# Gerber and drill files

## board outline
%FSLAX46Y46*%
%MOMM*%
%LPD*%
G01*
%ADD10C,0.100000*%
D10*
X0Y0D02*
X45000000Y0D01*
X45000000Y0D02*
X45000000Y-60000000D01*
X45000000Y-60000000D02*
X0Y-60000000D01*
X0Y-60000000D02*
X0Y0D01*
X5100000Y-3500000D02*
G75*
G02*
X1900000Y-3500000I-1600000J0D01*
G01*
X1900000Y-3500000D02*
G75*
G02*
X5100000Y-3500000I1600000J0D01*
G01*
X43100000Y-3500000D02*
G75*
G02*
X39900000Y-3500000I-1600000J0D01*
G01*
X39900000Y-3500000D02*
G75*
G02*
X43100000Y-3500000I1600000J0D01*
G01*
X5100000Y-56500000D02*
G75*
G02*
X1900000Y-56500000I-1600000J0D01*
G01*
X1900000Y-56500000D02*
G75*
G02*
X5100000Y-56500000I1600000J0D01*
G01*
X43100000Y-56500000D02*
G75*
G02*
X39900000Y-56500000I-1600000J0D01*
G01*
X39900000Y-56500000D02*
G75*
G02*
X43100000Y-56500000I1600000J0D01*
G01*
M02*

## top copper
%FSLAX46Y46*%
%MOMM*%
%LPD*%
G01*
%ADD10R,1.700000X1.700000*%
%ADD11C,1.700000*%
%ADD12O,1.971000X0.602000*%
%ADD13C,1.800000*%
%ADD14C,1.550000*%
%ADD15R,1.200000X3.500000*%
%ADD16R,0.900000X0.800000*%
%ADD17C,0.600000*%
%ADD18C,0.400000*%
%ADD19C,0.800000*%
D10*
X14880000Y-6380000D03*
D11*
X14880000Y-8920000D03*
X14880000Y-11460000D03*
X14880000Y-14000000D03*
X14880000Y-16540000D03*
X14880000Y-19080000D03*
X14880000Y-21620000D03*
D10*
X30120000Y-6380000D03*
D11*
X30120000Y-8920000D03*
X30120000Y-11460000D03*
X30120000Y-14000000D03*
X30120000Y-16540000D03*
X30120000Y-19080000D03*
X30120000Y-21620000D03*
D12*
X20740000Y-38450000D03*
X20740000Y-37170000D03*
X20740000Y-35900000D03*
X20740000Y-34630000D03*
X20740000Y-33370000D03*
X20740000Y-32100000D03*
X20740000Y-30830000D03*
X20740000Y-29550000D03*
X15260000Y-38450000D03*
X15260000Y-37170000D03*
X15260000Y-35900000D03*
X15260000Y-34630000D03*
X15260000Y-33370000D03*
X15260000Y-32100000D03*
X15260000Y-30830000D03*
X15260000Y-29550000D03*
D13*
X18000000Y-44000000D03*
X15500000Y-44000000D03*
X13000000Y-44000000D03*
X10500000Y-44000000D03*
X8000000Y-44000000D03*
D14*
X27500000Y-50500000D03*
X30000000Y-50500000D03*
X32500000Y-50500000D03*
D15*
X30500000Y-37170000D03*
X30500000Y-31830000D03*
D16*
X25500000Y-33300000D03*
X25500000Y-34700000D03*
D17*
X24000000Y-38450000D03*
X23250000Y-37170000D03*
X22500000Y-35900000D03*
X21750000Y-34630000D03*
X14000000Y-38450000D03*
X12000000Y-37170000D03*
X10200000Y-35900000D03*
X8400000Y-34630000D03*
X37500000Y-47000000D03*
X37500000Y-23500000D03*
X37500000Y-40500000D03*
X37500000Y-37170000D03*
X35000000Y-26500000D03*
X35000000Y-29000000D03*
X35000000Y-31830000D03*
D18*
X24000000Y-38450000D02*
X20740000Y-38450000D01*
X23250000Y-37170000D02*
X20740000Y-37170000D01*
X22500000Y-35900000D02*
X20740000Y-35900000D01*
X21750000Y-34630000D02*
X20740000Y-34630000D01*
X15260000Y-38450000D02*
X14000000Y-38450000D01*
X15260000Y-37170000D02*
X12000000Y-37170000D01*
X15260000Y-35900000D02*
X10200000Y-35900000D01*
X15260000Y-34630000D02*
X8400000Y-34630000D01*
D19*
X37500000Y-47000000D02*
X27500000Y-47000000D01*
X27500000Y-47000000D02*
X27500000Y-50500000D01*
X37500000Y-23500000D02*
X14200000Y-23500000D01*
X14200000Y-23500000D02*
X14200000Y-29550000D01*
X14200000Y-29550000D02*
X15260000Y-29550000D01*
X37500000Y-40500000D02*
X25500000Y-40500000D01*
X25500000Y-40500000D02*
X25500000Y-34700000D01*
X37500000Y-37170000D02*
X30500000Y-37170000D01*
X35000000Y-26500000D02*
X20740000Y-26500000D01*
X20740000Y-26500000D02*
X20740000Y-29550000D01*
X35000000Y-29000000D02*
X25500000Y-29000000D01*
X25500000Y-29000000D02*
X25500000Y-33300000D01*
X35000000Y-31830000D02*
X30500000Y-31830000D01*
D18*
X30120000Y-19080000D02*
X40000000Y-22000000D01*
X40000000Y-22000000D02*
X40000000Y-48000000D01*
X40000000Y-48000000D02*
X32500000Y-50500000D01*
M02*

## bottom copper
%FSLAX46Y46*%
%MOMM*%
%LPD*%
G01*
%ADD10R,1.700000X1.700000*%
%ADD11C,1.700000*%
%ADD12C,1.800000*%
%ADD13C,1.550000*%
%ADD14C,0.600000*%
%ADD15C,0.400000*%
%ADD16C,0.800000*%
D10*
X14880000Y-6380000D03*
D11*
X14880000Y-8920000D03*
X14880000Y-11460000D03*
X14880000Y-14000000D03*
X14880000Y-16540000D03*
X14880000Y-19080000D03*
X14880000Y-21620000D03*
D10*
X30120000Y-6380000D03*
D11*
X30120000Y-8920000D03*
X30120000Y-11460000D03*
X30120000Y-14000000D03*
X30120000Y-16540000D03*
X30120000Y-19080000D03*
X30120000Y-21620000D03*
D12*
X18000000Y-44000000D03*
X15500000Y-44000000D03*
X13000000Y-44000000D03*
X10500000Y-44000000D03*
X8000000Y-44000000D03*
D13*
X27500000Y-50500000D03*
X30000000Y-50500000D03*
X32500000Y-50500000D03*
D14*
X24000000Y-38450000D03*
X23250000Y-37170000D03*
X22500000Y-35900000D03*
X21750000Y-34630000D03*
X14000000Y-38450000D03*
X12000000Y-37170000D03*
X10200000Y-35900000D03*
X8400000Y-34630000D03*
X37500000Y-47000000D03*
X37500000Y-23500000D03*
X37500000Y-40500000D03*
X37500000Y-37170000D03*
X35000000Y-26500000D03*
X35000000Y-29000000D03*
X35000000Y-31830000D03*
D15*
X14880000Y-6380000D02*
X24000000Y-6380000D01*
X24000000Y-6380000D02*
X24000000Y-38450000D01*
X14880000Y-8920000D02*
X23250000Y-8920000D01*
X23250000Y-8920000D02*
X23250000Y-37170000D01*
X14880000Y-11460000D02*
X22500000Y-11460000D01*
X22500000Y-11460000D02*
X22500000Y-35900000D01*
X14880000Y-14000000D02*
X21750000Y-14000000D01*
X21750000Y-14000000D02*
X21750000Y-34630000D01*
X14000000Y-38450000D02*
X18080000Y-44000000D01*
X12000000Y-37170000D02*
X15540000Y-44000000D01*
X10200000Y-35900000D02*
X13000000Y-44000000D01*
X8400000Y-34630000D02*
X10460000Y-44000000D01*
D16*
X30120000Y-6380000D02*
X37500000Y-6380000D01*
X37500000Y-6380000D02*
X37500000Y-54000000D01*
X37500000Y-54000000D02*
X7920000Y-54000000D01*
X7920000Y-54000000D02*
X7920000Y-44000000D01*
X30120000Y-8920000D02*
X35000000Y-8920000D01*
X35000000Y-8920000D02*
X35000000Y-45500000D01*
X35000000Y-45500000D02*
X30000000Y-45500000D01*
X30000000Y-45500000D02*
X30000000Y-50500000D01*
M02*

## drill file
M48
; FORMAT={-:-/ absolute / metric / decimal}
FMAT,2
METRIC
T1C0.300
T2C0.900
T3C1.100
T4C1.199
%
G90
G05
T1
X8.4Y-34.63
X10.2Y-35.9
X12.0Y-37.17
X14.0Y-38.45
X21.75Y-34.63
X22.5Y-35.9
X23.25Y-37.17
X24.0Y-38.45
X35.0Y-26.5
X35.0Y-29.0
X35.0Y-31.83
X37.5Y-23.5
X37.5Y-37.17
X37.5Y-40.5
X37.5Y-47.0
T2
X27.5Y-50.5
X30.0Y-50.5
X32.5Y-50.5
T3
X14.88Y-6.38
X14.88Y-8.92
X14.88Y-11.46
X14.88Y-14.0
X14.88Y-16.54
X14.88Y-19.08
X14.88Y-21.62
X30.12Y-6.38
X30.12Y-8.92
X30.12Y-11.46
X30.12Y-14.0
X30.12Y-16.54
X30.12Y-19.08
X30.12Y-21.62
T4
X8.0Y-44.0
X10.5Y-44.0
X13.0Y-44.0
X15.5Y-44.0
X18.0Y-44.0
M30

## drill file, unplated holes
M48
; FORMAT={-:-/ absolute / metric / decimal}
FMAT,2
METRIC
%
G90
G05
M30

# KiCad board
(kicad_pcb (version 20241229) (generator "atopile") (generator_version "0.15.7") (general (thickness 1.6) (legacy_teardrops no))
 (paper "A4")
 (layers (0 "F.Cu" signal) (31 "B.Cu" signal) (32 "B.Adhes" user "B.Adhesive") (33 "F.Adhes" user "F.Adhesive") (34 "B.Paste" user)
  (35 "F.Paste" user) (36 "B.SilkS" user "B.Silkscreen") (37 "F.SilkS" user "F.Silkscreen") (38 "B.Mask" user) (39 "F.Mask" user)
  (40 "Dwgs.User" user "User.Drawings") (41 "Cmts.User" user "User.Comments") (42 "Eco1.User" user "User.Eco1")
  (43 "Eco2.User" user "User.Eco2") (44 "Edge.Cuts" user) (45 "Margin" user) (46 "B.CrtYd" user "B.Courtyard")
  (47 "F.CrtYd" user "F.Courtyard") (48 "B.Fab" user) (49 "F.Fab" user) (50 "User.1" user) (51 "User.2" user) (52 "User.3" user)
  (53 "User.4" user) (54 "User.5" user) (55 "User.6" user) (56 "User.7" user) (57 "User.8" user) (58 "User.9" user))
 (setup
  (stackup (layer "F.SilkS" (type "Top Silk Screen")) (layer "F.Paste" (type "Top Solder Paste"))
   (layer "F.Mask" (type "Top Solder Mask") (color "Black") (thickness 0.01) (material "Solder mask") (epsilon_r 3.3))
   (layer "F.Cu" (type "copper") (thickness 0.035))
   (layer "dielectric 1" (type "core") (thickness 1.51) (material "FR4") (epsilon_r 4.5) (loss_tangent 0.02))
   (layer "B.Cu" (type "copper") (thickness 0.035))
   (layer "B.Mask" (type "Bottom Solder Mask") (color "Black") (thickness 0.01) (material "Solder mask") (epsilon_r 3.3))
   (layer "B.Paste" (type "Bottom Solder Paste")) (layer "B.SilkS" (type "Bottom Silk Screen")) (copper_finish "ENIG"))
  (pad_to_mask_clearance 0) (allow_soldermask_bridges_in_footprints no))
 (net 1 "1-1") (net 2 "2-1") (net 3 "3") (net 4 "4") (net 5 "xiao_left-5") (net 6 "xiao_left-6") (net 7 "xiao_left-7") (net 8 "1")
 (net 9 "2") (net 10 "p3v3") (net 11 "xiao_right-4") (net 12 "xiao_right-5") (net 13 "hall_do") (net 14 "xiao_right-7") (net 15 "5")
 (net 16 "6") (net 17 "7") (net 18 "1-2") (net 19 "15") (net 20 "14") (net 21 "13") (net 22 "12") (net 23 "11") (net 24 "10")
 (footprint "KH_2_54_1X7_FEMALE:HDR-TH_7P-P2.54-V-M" (layer "F.Cu") (at 14.88 14 270)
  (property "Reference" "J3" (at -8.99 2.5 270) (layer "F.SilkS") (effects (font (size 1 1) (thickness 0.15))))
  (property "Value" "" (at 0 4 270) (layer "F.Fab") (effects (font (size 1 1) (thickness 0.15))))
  (pad "1" thru_hole rect (at -7.62 0 270) (size 1.7 1.7) (drill 1.100024) (layers "*.Cu" "*.Mask") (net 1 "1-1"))
  (pad "2" thru_hole circle (at -5.08 0 270) (size 1.7 1.7) (drill 1.100024) (layers "*.Cu" "*.Mask") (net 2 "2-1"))
  (pad "3" thru_hole circle (at -2.54 0 270) (size 1.7 1.7) (drill 1.100024) (layers "*.Cu" "*.Mask") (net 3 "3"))
  (pad "4" thru_hole circle (at 0 0 270) (size 1.7 1.7) (drill 1.100024) (layers "*.Cu" "*.Mask") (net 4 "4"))
  (pad "5" thru_hole circle (at 2.54 0 270) (size 1.7 1.7) (drill 1.100024) (layers "*.Cu" "*.Mask") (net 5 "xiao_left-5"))
  (pad "6" thru_hole circle (at 5.08 0 270) (size 1.7 1.7) (drill 1.100024) (layers "*.Cu" "*.Mask") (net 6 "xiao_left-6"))
  (pad "7" thru_hole circle (at 7.62 0 270) (size 1.7 1.7) (drill 1.100024) (layers "*.Cu" "*.Mask") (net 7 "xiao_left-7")))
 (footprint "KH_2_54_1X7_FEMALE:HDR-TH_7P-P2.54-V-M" (layer "F.Cu") (at 30.12 14 270)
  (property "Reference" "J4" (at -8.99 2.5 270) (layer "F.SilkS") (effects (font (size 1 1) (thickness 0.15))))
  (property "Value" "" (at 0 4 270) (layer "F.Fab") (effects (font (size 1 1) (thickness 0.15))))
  (pad "1" thru_hole rect (at -7.62 0 270) (size 1.7 1.7) (drill 1.100024) (layers "*.Cu" "*.Mask") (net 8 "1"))
  (pad "2" thru_hole circle (at -5.08 0 270) (size 1.7 1.7) (drill 1.100024) (layers "*.Cu" "*.Mask") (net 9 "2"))
  (pad "3" thru_hole circle (at -2.54 0 270) (size 1.7 1.7) (drill 1.100024) (layers "*.Cu" "*.Mask") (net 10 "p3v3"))
  (pad "4" thru_hole circle (at 0 0 270) (size 1.7 1.7) (drill 1.100024) (layers "*.Cu" "*.Mask") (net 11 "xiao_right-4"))
  (pad "5" thru_hole circle (at 2.54 0 270) (size 1.7 1.7) (drill 1.100024) (layers "*.Cu" "*.Mask") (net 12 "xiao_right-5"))
  (pad "6" thru_hole circle (at 5.08 0 270) (size 1.7 1.7) (drill 1.100024) (layers "*.Cu" "*.Mask") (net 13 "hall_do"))
  (pad "7" thru_hole circle (at 7.62 0 270) (size 1.7 1.7) (drill 1.100024) (layers "*.Cu" "*.Mask") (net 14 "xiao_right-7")))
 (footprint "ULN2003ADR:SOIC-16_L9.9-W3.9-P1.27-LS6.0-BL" (layer "F.Cu") (at 18 34 90)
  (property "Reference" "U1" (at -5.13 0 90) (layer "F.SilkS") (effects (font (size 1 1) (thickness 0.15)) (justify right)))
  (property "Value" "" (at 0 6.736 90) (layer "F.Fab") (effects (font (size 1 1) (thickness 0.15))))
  (pad "1" smd oval (at -4.45 2.74 90) (size 0.602 1.971) (layers "F.Cu" "F.Paste" "F.Mask") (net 1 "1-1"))
  (pad "2" smd oval (at -3.17 2.74 90) (size 0.602 1.971) (layers "F.Cu" "F.Paste" "F.Mask") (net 2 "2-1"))
  (pad "3" smd oval (at -1.9 2.74 90) (size 0.602 1.971) (layers "F.Cu" "F.Paste" "F.Mask") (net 3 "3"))
  (pad "4" smd oval (at -0.63 2.74 90) (size 0.602 1.971) (layers "F.Cu" "F.Paste" "F.Mask") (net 4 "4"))
  (pad "5" smd oval (at 0.63 2.74 90) (size 0.602 1.971) (layers "F.Cu" "F.Paste" "F.Mask") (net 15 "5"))
  (pad "6" smd oval (at 1.9 2.74 90) (size 0.602 1.971) (layers "F.Cu" "F.Paste" "F.Mask") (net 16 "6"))
  (pad "7" smd oval (at 3.17 2.74 90) (size 0.602 1.971) (layers "F.Cu" "F.Paste" "F.Mask") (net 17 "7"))
  (pad "8" smd oval (at 4.45 2.74 90) (size 0.602 1.971) (layers "F.Cu" "F.Paste" "F.Mask") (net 9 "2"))
  (pad "16" smd oval (at -4.45 -2.74 90) (size 0.602 1.971) (layers "F.Cu" "F.Paste" "F.Mask") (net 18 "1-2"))
  (pad "15" smd oval (at -3.17 -2.74 90) (size 0.602 1.971) (layers "F.Cu" "F.Paste" "F.Mask") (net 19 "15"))
  (pad "14" smd oval (at -1.9 -2.74 90) (size 0.602 1.971) (layers "F.Cu" "F.Paste" "F.Mask") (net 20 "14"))
  (pad "13" smd oval (at -0.63 -2.74 90) (size 0.602 1.971) (layers "F.Cu" "F.Paste" "F.Mask") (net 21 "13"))
  (pad "12" smd oval (at 0.63 -2.74 90) (size 0.602 1.971) (layers "F.Cu" "F.Paste" "F.Mask") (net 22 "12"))
  (pad "11" smd oval (at 1.9 -2.74 90) (size 0.602 1.971) (layers "F.Cu" "F.Paste" "F.Mask") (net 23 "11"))
  (pad "10" smd oval (at 3.17 -2.74 90) (size 0.602 1.971) (layers "F.Cu" "F.Paste" "F.Mask") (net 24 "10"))
  (pad "9" smd oval (at 4.45 -2.74 90) (size 0.602 1.971) (layers "F.Cu" "F.Paste" "F.Mask") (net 8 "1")))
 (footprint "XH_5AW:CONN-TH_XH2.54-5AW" (layer "F.Cu") (at 13 44 0)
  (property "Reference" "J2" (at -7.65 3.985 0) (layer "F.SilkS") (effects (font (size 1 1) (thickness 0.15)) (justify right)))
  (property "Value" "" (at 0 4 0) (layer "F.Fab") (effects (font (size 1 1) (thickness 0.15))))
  (pad "1" thru_hole circle (at 5 -0 180) (size 1.8 1.8) (drill 1.19888) (layers "*.Cu" "*.Mask") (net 18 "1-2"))
  (pad "2" thru_hole circle (at 2.5 -0 180) (size 1.8 1.8) (drill 1.19888) (layers "*.Cu" "*.Mask") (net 19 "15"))
  (pad "3" thru_hole circle (at -0 -0 180) (size 1.8 1.8) (drill 1.19888) (layers "*.Cu" "*.Mask") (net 20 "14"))
  (pad "4" thru_hole circle (at -2.5 -0 180) (size 1.8 1.8) (drill 1.19888) (layers "*.Cu" "*.Mask") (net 21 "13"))
  (pad "5" thru_hole circle (at -5 -0 180) (size 1.8 1.8) (drill 1.19888) (layers "*.Cu" "*.Mask") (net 8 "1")))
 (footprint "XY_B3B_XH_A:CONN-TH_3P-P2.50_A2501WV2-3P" (layer "F.Cu") (at 30 50.5 0)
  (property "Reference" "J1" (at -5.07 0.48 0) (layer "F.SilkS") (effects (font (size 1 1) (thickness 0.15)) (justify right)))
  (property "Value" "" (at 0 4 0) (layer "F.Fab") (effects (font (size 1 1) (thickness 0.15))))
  (pad "1" thru_hole circle (at -2.5 0 180) (size 1.55 1.55) (drill 0.900024) (layers "*.Cu" "*.Mask") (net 8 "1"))
  (pad "2" thru_hole circle (at 0 0 180) (size 1.55 1.55) (drill 0.900024) (layers "*.Cu" "*.Mask") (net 9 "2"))
  (pad "3" thru_hole circle (at 2.5 0 180) (size 1.55 1.55) (drill 0.900024) (layers "*.Cu" "*.Mask") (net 13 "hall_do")))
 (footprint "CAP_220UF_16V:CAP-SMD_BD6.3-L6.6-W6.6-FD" (layer "F.Cu") (at 30.5 34.5 90)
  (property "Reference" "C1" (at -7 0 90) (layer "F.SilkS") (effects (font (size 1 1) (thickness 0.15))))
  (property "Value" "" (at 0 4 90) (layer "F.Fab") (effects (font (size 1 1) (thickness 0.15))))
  (pad "1" smd rect (at -2.67 0 90) (size 3.5 1.2) (layers "F.Cu" "F.Paste" "F.Mask") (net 8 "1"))
  (pad "2" smd rect (at 2.67 0 90) (size 3.5 1.2) (layers "F.Cu" "F.Paste" "F.Mask") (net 9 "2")))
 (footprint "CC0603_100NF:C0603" (layer "F.Cu") (at 25.5 34 90)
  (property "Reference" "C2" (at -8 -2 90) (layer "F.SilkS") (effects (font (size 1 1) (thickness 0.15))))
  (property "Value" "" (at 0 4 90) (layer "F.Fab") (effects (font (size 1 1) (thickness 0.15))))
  (pad "2" smd rect (at 0.7 0 90) (size 0.8 0.9) (layers "F.Cu" "F.Paste" "F.Mask") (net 9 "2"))
  (pad "1" smd rect (at -0.7 0 90) (size 0.8 0.9) (layers "F.Cu" "F.Paste" "F.Mask") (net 8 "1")))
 (via (at 24 38.45) (size 0.6) (drill 0.3) (layers "F.Cu" "B.Cu") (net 1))
 (via (at 23.25 37.17) (size 0.6) (drill 0.3) (layers "F.Cu" "B.Cu") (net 2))
 (via (at 22.5 35.9) (size 0.6) (drill 0.3) (layers "F.Cu" "B.Cu") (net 3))
 (via (at 21.75 34.63) (size 0.6) (drill 0.3) (layers "F.Cu" "B.Cu") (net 4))
 (via (at 14 38.45) (size 0.6) (drill 0.3) (layers "F.Cu" "B.Cu") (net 18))
 (via (at 12 37.17) (size 0.6) (drill 0.3) (layers "F.Cu" "B.Cu") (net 19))
 (via (at 10.2 35.9) (size 0.6) (drill 0.3) (layers "F.Cu" "B.Cu") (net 20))
 (via (at 8.4 34.63) (size 0.6) (drill 0.3) (layers "F.Cu" "B.Cu") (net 21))
 (via (at 37.5 47) (size 0.6) (drill 0.3) (layers "F.Cu" "B.Cu") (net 8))
 (via (at 37.5 23.5) (size 0.6) (drill 0.3) (layers "F.Cu" "B.Cu") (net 8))
 (via (at 37.5 40.5) (size 0.6) (drill 0.3) (layers "F.Cu" "B.Cu") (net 8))
 (via (at 37.5 37.17) (size 0.6) (drill 0.3) (layers "F.Cu" "B.Cu") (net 8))
 (via (at 35 26.5) (size 0.6) (drill 0.3) (layers "F.Cu" "B.Cu") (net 9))
 (via (at 35 29) (size 0.6) (drill 0.3) (layers "F.Cu" "B.Cu") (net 9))
 (via (at 35 31.83) (size 0.6) (drill 0.3) (layers "F.Cu" "B.Cu") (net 9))
 (segment (start 14.88 6.38) (end 24 6.38) (width 0.4) (layer "B.Cu") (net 1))
 (segment (start 24 6.38) (end 24 38.45) (width 0.4) (layer "B.Cu") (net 1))
 (segment (start 24 38.45) (end 20.74 38.45) (width 0.4) (layer "F.Cu") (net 1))
 (segment (start 14.88 8.92) (end 23.25 8.92) (width 0.4) (layer "B.Cu") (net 2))
 (segment (start 23.25 8.92) (end 23.25 37.17) (width 0.4) (layer "B.Cu") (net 2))
 (segment (start 23.25 37.17) (end 20.74 37.17) (width 0.4) (layer "F.Cu") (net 2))
 (segment (start 14.88 11.46) (end 22.5 11.46) (width 0.4) (layer "B.Cu") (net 3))
 (segment (start 22.5 11.46) (end 22.5 35.9) (width 0.4) (layer "B.Cu") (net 3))
 (segment (start 22.5 35.9) (end 20.74 35.9) (width 0.4) (layer "F.Cu") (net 3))
 (segment (start 14.88 14) (end 21.75 14) (width 0.4) (layer "B.Cu") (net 4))
 (segment (start 21.75 14) (end 21.75 34.63) (width 0.4) (layer "B.Cu") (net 4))
 (segment (start 21.75 34.63) (end 20.74 34.63) (width 0.4) (layer "F.Cu") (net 4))
 (segment (start 15.26 38.45) (end 14 38.45) (width 0.4) (layer "F.Cu") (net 18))
 (segment (start 14 38.45) (end 18.08 44) (width 0.4) (layer "B.Cu") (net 18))
 (segment (start 15.26 37.17) (end 12 37.17) (width 0.4) (layer "F.Cu") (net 19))
 (segment (start 12 37.17) (end 15.54 44) (width 0.4) (layer "B.Cu") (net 19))
 (segment (start 15.26 35.9) (end 10.2 35.9) (width 0.4) (layer "F.Cu") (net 20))
 (segment (start 10.2 35.9) (end 13 44) (width 0.4) (layer "B.Cu") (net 20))
 (segment (start 15.26 34.63) (end 8.4 34.63) (width 0.4) (layer "F.Cu") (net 21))
 (segment (start 8.4 34.63) (end 10.46 44) (width 0.4) (layer "B.Cu") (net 21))
 (segment (start 30.12 6.38) (end 37.5 6.38) (width 0.8) (layer "B.Cu") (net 8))
 (segment (start 37.5 6.38) (end 37.5 54) (width 0.8) (layer "B.Cu") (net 8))
 (segment (start 37.5 54) (end 7.92 54) (width 0.8) (layer "B.Cu") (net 8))
 (segment (start 7.92 54) (end 7.92 44) (width 0.8) (layer "B.Cu") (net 8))
 (segment (start 37.5 47) (end 27.5 47) (width 0.8) (layer "F.Cu") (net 8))
 (segment (start 27.5 47) (end 27.5 50.5) (width 0.8) (layer "F.Cu") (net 8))
 (segment (start 37.5 23.5) (end 14.2 23.5) (width 0.8) (layer "F.Cu") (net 8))
 (segment (start 14.2 23.5) (end 14.2 29.55) (width 0.8) (layer "F.Cu") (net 8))
 (segment (start 14.2 29.55) (end 15.26 29.55) (width 0.8) (layer "F.Cu") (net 8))
 (segment (start 37.5 40.5) (end 25.5 40.5) (width 0.8) (layer "F.Cu") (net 8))
 (segment (start 25.5 40.5) (end 25.5 34.7) (width 0.8) (layer "F.Cu") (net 8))
 (segment (start 37.5 37.17) (end 30.5 37.17) (width 0.8) (layer "F.Cu") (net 8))
 (segment (start 30.12 8.92) (end 35 8.92) (width 0.8) (layer "B.Cu") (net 9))
 (segment (start 35 8.92) (end 35 45.5) (width 0.8) (layer "B.Cu") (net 9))
 (segment (start 35 45.5) (end 30 45.5) (width 0.8) (layer "B.Cu") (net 9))
 (segment (start 30 45.5) (end 30 50.5) (width 0.8) (layer "B.Cu") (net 9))
 (segment (start 35 26.5) (end 20.74 26.5) (width 0.8) (layer "F.Cu") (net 9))
 (segment (start 20.74 26.5) (end 20.74 29.55) (width 0.8) (layer "F.Cu") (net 9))
 (segment (start 35 29) (end 25.5 29) (width 0.8) (layer "F.Cu") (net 9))
 (segment (start 25.5 29) (end 25.5 33.3) (width 0.8) (layer "F.Cu") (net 9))
 (segment (start 35 31.83) (end 30.5 31.83) (width 0.8) (layer "F.Cu") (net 9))
 (segment (start 30.12 19.08) (end 40 22) (width 0.4) (layer "F.Cu") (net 13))
 (segment (start 40 22) (end 40 48) (width 0.4) (layer "F.Cu") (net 13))
 (segment (start 40 48) (end 32.5 50.5) (width 0.4) (layer "F.Cu") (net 13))
 (gr_line (start 0 0) (end 45 0) (stroke (width 0.1) (type default)) (layer "Edge.Cuts"))
 (gr_line (start 45 0) (end 45 60) (stroke (width 0.1) (type default)) (layer "Edge.Cuts"))
 (gr_line (start 45 60) (end 0 60) (stroke (width 0.1) (type default)) (layer "Edge.Cuts"))
 (gr_line (start 0 60) (end 0 0) (stroke (width 0.1) (type default)) (layer "Edge.Cuts"))
 (gr_circle (center 3.5 3.5) (end 5.1 3.5) (stroke (width 0.1) (type default)) (fill none) (layer "Edge.Cuts"))
 (gr_circle (center 41.5 3.5) (end 43.1 3.5) (stroke (width 0.1) (type default)) (fill none) (layer "Edge.Cuts"))
 (gr_circle (center 3.5 56.5) (end 5.1 56.5) (stroke (width 0.1) (type default)) (fill none) (layer "Edge.Cuts"))
 (gr_circle (center 41.5 56.5) (end 43.1 56.5) (stroke (width 0.1) (type default)) (fill none) (layer "Edge.Cuts")))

